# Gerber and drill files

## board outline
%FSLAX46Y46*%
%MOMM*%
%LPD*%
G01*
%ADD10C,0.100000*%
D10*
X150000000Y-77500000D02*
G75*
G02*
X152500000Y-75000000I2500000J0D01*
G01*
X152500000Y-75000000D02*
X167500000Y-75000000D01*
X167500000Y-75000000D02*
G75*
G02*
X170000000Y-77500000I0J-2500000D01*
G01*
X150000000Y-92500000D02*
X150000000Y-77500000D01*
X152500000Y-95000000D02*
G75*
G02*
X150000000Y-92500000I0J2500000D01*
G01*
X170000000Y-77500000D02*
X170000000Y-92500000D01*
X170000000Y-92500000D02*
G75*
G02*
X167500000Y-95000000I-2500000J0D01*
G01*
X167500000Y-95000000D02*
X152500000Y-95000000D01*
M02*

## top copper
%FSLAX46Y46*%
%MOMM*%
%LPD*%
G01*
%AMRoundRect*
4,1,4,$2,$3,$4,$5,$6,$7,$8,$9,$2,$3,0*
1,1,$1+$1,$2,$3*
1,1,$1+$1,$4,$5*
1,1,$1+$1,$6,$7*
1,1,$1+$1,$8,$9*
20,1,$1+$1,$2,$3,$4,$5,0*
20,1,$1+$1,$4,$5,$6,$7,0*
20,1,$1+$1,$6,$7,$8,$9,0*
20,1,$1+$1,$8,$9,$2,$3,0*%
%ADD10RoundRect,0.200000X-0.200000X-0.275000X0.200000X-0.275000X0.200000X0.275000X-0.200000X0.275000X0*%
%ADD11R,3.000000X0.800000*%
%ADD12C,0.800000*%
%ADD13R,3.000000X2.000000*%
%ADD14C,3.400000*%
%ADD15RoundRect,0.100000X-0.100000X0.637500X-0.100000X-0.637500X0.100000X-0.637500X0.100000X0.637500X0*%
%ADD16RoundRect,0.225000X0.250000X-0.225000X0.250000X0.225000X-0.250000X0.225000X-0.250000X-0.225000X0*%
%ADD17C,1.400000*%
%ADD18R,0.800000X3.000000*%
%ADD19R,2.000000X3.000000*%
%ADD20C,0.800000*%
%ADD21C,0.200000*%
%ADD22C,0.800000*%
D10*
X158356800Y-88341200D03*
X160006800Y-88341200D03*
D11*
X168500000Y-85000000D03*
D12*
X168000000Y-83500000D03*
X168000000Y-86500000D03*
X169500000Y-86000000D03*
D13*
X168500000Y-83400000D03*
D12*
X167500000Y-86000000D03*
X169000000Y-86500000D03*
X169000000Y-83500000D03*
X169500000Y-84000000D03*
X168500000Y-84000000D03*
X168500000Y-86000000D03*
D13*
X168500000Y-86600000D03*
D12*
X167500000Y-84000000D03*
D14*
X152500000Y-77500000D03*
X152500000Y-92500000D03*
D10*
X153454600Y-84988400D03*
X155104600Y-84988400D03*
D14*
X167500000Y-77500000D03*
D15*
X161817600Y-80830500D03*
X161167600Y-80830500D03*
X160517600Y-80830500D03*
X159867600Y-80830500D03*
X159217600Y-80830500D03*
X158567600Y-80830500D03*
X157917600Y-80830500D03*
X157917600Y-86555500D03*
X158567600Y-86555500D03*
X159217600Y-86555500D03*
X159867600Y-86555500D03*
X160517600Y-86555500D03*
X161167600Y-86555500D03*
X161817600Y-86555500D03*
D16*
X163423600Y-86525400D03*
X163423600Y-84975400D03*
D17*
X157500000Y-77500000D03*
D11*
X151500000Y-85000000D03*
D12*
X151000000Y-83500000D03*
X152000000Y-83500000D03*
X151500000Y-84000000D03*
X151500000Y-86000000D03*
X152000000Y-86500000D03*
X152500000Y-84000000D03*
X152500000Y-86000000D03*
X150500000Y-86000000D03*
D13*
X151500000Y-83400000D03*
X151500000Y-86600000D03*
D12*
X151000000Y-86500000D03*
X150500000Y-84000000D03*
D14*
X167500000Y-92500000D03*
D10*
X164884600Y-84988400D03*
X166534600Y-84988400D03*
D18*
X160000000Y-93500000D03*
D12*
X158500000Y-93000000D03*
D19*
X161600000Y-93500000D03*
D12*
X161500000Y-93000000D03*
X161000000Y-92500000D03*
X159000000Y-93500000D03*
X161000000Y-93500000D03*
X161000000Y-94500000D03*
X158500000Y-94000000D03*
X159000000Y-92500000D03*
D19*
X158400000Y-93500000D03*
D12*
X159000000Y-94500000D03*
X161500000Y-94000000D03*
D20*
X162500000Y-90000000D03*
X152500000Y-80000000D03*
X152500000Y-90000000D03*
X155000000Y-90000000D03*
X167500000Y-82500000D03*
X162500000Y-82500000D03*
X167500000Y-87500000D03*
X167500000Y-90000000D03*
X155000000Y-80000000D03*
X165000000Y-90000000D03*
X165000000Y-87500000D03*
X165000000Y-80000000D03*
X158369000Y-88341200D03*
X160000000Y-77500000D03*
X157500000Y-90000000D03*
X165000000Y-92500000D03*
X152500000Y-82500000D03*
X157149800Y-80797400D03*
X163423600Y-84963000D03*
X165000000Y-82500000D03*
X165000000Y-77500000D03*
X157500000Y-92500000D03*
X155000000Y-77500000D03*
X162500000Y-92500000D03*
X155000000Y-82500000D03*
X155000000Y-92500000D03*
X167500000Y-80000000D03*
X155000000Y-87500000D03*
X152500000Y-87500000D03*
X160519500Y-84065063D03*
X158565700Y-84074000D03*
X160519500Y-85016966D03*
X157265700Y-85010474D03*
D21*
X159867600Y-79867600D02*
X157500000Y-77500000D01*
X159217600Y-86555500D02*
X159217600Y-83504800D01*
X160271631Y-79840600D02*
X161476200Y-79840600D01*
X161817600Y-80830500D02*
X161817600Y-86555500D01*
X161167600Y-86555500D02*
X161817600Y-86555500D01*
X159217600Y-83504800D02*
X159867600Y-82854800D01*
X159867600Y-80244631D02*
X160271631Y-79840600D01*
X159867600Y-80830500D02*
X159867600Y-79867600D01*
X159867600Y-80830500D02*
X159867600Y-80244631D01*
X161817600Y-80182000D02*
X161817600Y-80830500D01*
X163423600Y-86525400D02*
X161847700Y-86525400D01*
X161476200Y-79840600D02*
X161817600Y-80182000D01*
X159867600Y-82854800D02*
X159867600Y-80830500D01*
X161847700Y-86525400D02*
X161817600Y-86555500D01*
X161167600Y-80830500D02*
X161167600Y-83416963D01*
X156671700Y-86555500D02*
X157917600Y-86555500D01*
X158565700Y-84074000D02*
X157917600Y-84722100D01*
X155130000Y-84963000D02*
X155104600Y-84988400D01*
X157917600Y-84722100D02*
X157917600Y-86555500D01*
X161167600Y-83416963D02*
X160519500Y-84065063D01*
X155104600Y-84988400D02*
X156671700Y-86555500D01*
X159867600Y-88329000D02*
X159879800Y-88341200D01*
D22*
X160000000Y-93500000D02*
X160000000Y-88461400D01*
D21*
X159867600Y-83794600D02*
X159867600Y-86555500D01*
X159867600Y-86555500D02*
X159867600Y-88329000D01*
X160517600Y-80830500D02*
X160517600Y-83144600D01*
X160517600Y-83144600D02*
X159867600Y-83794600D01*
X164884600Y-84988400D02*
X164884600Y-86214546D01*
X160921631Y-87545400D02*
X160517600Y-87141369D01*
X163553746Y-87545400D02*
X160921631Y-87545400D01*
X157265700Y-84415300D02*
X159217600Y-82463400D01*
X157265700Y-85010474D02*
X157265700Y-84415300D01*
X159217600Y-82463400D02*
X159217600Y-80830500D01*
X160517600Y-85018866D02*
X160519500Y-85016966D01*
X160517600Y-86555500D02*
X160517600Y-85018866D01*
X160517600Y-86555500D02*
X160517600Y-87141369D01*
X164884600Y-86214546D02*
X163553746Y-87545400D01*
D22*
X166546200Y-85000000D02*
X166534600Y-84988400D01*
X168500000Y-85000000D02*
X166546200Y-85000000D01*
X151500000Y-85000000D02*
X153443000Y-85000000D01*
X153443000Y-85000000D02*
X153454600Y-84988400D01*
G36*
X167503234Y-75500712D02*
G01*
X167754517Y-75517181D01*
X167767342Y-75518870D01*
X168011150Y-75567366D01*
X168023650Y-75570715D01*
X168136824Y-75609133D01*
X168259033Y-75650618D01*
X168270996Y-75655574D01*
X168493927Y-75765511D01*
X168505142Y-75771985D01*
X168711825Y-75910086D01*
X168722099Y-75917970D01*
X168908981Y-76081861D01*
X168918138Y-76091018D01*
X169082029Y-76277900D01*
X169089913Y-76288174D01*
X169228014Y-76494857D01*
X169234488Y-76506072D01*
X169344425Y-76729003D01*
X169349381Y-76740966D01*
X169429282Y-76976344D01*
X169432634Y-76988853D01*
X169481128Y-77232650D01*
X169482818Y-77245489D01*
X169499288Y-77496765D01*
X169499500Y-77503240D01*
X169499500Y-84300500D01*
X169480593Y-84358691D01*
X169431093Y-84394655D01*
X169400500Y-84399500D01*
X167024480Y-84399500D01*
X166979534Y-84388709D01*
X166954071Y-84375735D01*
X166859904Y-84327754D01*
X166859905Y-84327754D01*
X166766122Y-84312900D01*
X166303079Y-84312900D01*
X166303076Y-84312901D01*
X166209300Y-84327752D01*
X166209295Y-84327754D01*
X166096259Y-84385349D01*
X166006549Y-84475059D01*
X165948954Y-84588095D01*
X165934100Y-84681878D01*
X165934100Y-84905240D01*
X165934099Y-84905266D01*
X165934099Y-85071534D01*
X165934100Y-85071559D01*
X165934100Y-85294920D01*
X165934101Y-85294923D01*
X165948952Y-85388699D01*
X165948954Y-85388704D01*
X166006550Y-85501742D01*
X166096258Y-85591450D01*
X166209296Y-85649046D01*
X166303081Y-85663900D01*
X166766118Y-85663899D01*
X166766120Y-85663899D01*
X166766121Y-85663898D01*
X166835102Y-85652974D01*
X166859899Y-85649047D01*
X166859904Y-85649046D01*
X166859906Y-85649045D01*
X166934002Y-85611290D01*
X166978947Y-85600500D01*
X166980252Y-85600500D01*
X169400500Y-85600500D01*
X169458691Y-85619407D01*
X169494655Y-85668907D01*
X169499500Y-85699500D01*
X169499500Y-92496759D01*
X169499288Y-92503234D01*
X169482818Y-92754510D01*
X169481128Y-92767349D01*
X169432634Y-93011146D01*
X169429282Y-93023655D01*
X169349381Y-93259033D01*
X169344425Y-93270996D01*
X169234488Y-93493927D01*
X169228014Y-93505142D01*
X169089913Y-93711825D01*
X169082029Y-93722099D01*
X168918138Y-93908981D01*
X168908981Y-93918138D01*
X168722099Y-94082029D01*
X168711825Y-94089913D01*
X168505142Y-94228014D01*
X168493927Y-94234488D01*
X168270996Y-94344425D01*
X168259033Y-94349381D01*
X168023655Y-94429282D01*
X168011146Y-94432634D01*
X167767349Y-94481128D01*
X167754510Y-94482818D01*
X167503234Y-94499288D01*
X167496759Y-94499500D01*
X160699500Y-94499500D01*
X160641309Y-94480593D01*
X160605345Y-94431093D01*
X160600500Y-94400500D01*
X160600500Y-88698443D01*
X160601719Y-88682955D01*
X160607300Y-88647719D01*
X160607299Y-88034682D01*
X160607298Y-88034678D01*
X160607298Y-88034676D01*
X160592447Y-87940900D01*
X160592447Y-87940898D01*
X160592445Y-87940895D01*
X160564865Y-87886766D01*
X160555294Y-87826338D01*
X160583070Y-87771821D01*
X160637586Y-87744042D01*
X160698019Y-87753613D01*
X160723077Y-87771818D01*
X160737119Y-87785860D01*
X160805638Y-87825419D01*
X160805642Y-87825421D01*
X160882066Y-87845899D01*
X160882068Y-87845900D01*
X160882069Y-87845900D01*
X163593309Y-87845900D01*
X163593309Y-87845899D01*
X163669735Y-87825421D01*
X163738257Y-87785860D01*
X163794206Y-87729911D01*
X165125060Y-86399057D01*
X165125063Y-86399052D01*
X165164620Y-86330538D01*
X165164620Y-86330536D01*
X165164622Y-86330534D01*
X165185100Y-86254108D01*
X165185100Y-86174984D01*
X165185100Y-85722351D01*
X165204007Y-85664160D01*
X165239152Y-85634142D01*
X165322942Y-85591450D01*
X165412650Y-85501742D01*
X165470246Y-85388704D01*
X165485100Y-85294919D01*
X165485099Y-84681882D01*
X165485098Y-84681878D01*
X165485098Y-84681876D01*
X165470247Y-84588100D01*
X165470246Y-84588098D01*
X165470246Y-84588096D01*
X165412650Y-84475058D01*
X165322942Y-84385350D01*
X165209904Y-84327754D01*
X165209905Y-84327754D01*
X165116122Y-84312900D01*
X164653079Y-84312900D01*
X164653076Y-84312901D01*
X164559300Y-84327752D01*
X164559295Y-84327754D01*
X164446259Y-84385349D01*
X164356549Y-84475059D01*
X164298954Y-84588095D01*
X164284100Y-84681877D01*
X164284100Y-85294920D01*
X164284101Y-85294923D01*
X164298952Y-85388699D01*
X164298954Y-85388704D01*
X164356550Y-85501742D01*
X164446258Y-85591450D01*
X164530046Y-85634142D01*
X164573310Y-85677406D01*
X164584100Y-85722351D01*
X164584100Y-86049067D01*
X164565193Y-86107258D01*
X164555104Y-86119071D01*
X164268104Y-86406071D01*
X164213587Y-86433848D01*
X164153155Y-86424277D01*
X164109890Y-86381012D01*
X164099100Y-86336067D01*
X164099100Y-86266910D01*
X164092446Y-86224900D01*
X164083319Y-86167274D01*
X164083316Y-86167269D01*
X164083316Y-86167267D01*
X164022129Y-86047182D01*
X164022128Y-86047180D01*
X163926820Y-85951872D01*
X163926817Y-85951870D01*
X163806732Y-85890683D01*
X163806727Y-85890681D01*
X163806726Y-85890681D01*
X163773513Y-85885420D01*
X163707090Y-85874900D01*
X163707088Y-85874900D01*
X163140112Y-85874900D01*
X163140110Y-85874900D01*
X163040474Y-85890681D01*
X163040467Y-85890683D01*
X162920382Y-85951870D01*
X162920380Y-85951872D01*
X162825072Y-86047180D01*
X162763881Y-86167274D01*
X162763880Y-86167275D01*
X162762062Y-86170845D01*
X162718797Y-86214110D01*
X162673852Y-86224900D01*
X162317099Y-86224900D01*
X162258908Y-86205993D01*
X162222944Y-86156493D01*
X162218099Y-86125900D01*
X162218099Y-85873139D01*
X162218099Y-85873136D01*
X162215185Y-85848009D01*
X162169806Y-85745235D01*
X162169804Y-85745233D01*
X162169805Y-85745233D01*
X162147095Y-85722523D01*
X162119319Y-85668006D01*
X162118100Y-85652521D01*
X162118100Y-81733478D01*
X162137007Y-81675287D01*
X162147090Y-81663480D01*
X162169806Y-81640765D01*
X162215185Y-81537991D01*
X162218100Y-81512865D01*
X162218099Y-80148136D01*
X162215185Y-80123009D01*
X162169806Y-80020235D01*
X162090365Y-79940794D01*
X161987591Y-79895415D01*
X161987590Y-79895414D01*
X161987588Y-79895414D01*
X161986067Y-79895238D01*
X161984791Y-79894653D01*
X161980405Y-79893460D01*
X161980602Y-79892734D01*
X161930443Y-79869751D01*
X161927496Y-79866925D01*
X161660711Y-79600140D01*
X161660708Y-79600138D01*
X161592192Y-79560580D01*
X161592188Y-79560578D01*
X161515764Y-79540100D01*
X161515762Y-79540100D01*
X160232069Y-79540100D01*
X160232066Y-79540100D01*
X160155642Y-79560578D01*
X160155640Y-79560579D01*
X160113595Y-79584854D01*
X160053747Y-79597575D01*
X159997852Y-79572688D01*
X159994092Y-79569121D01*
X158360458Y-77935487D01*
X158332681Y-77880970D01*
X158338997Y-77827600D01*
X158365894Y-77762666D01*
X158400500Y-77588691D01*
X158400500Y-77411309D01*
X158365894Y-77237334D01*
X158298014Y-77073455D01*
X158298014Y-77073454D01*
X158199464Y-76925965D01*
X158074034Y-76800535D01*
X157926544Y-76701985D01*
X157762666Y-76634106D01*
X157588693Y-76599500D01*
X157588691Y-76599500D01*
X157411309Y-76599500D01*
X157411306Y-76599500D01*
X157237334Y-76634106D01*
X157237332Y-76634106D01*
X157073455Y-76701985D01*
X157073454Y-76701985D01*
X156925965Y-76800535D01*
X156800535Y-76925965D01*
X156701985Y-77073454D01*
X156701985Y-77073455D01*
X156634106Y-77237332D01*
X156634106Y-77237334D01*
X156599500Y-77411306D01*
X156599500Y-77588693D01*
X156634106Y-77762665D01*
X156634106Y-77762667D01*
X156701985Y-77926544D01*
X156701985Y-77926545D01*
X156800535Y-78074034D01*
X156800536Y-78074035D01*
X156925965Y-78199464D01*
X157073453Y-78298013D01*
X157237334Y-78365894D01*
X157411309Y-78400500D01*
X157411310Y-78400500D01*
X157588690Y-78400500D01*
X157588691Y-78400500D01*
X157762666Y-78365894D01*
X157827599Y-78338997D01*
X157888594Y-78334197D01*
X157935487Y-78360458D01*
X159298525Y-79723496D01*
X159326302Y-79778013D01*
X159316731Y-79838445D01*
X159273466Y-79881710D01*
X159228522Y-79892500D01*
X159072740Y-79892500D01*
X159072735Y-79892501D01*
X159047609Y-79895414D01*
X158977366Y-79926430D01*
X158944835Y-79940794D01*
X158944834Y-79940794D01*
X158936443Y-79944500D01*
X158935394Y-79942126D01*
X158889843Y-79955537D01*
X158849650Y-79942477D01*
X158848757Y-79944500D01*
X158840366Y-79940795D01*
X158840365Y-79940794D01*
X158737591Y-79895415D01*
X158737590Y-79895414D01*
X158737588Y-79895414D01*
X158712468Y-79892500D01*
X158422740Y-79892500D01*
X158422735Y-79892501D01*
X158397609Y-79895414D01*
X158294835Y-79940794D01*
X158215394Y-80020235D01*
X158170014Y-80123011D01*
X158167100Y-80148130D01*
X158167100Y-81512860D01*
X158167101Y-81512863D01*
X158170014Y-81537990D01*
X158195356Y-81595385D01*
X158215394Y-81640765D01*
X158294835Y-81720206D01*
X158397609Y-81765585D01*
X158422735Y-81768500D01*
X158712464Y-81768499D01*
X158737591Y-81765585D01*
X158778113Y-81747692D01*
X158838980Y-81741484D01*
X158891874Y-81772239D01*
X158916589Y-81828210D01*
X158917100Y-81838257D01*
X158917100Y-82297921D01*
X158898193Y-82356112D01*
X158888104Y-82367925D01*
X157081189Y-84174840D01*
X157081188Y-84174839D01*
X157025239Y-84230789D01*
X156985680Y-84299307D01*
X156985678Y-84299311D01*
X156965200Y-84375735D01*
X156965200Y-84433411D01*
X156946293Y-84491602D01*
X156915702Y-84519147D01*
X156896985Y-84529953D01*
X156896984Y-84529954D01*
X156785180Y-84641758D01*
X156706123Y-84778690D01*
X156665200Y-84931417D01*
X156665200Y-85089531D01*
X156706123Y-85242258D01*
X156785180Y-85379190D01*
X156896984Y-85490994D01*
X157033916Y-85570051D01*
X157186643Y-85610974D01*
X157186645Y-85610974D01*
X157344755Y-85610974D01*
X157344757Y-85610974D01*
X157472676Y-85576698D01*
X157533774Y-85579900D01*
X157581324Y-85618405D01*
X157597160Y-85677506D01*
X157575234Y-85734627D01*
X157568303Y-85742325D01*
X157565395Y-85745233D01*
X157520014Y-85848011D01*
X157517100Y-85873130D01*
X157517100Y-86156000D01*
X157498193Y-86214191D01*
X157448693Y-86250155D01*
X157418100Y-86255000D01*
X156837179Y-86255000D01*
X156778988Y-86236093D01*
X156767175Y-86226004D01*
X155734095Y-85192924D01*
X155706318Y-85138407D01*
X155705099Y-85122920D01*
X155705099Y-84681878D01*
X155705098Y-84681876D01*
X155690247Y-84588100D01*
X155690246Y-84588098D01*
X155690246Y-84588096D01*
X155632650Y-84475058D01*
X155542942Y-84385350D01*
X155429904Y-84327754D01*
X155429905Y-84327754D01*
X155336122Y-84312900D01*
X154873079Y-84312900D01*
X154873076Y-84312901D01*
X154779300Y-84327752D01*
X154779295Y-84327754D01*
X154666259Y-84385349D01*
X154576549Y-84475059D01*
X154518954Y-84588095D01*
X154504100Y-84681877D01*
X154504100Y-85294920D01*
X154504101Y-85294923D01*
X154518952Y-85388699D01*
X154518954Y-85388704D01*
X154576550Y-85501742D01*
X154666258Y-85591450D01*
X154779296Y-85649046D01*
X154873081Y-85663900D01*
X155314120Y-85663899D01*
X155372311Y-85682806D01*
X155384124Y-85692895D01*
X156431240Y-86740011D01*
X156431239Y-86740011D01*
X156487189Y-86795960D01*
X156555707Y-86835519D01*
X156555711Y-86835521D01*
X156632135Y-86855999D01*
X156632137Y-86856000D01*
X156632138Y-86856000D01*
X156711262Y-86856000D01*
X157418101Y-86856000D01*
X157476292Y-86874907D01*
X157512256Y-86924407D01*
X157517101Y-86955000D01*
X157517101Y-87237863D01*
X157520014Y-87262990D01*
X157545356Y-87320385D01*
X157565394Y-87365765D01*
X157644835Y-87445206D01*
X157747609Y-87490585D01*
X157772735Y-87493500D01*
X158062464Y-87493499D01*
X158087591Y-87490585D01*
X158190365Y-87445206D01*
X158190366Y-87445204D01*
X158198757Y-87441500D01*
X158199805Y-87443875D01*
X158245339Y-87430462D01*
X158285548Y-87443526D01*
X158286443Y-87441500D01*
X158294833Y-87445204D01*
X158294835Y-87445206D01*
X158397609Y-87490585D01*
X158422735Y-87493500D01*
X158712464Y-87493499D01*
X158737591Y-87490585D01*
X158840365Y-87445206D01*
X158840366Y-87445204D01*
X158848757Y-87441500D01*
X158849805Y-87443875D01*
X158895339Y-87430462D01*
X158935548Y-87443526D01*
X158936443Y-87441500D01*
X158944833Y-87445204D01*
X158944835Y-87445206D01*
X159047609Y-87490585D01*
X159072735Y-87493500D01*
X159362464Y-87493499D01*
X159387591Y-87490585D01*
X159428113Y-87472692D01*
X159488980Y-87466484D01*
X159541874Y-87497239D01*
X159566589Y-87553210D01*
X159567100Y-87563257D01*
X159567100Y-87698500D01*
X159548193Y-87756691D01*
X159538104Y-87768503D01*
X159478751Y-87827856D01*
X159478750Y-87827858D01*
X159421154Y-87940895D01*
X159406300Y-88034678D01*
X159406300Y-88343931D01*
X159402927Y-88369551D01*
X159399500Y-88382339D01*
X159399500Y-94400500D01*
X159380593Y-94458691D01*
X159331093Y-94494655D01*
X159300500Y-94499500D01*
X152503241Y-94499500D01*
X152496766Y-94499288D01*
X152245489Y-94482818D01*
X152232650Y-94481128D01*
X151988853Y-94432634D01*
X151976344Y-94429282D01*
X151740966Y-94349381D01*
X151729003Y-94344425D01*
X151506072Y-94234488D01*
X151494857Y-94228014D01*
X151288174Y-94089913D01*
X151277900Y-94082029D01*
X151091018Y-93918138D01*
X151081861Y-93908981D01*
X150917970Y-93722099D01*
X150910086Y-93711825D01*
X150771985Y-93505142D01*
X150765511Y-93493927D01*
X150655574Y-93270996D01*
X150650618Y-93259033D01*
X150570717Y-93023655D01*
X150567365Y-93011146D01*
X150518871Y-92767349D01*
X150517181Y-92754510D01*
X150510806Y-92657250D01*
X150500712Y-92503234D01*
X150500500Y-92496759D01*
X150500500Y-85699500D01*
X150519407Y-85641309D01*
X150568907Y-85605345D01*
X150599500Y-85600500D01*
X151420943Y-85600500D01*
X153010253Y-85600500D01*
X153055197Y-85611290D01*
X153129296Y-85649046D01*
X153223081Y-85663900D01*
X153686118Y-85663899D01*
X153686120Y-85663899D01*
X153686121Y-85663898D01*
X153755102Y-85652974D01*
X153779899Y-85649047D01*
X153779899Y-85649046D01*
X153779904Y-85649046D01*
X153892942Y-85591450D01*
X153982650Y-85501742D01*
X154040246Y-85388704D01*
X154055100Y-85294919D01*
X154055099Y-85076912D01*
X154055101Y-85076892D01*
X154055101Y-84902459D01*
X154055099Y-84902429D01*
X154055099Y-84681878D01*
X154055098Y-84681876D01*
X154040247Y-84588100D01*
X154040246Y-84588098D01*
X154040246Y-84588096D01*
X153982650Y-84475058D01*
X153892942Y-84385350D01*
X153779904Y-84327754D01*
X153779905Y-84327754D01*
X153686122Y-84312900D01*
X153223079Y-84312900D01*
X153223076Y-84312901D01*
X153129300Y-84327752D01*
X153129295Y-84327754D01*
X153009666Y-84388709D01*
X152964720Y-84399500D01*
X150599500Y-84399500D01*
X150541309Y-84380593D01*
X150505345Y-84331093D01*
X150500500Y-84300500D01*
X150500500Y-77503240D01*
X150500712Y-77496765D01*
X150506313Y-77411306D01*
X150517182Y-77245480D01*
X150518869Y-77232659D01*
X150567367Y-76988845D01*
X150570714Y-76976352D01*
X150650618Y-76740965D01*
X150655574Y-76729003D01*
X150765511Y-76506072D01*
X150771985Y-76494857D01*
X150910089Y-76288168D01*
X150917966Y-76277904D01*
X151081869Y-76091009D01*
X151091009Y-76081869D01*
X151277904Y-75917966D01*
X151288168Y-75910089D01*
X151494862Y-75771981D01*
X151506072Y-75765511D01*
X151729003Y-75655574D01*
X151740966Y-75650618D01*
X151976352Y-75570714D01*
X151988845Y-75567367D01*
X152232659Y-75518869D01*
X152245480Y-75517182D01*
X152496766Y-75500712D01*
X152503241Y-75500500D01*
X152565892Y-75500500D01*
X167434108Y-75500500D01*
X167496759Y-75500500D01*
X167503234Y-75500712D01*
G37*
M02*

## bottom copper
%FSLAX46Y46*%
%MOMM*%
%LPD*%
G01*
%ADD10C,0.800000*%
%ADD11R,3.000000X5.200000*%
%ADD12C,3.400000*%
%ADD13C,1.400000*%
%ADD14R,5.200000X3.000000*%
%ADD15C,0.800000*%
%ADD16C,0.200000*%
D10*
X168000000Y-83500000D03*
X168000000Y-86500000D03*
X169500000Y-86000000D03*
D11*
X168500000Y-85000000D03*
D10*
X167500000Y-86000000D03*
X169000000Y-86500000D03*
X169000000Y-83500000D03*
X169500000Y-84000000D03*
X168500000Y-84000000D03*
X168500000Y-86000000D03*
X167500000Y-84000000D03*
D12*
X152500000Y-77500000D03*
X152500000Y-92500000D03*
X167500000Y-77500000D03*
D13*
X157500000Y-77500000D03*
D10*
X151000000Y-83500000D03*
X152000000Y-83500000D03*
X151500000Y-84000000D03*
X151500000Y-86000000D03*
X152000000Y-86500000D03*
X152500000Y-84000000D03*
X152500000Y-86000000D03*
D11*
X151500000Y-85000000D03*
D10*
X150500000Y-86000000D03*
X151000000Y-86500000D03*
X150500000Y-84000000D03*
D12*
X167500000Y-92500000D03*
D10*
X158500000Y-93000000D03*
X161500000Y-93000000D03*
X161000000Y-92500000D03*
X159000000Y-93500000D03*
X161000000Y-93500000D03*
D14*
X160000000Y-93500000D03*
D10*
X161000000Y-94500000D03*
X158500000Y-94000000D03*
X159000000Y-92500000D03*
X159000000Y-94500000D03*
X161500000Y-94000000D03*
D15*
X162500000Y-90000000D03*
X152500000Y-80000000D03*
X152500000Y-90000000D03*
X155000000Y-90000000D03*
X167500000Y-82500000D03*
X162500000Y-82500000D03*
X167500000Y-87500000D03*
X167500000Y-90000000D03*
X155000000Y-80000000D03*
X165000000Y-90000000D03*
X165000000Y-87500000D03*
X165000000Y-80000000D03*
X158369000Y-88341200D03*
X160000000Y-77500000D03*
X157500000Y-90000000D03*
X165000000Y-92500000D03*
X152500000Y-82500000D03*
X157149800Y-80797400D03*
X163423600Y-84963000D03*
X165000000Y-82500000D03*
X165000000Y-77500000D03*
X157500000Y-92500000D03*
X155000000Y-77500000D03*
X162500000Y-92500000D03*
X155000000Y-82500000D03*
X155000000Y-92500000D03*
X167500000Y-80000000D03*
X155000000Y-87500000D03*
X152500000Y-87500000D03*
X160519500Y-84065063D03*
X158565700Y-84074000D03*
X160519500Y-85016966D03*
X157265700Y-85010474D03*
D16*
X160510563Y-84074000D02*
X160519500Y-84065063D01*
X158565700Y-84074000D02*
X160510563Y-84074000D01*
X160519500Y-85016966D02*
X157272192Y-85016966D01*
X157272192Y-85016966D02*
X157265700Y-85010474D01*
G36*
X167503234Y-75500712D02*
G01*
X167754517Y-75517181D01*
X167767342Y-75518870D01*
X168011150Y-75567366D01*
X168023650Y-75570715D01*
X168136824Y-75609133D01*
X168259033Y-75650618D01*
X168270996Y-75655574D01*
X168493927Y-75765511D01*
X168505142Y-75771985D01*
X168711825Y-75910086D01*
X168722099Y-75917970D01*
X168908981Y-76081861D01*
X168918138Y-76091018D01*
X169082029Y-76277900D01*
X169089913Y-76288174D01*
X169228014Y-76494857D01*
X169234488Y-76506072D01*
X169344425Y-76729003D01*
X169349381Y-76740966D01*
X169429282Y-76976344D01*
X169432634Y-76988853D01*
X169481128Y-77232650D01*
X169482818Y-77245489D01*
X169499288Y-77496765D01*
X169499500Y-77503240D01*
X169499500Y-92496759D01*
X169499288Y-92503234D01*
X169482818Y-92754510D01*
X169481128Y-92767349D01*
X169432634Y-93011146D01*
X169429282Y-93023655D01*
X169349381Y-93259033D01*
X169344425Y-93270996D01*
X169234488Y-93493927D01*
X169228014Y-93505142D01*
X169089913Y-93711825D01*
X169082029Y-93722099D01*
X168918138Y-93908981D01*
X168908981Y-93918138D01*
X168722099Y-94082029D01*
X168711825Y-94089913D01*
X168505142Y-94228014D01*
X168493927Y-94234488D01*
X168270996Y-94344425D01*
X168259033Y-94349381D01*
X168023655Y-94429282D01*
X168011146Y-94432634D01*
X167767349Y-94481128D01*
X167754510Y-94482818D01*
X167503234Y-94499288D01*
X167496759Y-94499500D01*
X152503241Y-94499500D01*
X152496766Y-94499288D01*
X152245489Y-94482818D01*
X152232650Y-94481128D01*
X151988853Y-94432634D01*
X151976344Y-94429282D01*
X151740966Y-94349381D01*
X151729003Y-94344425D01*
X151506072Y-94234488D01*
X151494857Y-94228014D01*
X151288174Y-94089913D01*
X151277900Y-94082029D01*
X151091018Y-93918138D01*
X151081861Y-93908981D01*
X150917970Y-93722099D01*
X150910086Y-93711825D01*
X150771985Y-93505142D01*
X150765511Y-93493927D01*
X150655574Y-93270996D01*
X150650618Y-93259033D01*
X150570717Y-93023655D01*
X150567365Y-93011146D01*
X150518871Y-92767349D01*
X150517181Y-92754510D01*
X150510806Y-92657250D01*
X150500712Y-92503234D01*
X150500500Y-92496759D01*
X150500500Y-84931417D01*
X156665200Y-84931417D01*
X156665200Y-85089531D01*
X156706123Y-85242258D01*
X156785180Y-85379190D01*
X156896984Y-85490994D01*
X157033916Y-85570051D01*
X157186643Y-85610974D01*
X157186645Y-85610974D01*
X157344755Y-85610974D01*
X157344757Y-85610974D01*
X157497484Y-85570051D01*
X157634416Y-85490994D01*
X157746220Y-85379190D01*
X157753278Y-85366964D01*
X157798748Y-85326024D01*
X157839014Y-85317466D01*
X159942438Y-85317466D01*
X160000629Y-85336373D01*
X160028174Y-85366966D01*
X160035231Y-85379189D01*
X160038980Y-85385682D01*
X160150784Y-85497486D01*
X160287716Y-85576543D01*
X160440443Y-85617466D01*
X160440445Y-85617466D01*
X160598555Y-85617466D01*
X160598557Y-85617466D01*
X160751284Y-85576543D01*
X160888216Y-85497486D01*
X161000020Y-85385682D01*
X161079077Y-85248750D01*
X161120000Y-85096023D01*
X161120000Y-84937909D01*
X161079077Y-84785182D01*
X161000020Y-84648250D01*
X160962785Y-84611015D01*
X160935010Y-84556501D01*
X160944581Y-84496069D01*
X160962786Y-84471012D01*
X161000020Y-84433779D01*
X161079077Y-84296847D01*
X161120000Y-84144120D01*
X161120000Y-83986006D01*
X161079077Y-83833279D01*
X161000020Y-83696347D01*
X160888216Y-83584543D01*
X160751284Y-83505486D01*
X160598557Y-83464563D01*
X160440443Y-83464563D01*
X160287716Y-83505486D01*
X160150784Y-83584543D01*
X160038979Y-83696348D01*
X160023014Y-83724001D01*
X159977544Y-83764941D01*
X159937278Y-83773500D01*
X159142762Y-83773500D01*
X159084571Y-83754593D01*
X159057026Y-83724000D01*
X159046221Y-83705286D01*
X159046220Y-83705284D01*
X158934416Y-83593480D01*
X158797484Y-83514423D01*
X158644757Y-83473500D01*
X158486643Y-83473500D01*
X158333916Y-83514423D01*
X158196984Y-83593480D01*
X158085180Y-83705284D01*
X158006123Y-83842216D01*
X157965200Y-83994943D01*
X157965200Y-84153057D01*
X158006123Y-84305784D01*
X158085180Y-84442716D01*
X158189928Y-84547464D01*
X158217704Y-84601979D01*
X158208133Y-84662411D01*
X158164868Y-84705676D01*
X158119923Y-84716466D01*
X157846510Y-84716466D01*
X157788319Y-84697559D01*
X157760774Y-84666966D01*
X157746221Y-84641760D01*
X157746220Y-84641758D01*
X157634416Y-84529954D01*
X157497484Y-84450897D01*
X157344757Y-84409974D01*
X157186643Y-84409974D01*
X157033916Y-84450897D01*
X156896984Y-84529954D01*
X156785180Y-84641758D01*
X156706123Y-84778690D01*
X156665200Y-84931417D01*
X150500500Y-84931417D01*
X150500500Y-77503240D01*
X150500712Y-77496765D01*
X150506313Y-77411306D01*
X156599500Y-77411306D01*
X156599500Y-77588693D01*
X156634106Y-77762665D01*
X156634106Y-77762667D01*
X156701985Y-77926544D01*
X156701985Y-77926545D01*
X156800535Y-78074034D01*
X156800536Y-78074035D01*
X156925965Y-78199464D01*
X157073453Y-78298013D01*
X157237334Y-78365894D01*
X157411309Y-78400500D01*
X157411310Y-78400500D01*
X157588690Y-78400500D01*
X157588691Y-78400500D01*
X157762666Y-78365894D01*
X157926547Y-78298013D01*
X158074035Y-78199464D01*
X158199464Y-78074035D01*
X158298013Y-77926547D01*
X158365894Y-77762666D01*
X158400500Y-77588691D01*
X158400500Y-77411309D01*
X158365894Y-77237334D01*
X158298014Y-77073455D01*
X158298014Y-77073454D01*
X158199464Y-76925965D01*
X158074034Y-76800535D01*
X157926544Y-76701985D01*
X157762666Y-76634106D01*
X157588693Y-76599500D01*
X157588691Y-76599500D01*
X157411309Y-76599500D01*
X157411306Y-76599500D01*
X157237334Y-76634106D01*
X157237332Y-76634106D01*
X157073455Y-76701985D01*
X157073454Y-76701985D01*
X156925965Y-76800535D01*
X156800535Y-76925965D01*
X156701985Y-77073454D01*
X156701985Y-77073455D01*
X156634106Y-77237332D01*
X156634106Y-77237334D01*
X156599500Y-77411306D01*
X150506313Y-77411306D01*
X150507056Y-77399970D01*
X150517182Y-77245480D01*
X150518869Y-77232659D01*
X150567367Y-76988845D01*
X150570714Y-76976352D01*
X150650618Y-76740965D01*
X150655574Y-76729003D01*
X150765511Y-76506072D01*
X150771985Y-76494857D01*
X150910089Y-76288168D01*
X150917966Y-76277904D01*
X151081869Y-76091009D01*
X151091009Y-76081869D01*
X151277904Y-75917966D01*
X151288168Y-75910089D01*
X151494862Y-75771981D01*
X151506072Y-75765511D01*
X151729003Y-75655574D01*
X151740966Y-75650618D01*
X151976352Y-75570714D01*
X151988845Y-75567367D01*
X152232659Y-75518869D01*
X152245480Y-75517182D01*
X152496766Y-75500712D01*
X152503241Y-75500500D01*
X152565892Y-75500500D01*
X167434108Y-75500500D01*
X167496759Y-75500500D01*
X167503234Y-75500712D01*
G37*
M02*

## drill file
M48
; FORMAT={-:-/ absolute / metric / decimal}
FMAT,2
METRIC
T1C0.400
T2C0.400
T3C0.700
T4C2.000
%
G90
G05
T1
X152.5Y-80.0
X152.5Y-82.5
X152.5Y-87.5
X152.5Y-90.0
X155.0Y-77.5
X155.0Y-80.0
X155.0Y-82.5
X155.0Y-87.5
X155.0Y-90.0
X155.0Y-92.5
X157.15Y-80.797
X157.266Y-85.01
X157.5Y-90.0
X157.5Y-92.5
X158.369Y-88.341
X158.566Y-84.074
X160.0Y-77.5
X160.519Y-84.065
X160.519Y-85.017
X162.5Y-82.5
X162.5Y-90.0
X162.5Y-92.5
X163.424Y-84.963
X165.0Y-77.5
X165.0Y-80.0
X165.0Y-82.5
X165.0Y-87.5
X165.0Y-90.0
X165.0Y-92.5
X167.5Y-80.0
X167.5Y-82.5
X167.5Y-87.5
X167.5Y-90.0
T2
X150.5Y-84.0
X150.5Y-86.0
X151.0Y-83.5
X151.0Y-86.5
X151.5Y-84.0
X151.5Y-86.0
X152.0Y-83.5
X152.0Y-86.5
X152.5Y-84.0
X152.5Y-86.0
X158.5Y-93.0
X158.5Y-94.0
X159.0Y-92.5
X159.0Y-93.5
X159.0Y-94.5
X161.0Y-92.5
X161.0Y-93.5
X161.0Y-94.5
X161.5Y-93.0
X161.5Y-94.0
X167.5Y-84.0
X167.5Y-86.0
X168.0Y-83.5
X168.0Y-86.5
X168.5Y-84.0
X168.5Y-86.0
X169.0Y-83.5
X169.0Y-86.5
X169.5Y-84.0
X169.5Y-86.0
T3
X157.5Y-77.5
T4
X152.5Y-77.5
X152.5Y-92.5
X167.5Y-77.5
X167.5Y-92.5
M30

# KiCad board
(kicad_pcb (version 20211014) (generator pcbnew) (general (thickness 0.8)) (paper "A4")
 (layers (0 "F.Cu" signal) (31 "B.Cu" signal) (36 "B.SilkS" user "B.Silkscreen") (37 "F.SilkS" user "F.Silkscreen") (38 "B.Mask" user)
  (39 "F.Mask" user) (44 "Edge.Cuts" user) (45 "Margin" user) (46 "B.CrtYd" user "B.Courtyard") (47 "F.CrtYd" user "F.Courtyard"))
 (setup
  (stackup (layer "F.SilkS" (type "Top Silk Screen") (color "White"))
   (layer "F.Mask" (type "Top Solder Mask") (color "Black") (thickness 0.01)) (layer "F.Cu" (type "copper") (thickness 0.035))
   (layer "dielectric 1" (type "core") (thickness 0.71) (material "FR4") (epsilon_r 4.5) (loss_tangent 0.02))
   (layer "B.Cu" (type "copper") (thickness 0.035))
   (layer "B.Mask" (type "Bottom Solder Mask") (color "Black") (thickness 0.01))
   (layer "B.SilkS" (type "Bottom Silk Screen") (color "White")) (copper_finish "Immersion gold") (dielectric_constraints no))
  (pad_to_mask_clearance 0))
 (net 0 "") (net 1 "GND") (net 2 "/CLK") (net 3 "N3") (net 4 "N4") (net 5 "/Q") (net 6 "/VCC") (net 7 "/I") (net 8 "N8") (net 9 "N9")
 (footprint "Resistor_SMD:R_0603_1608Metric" (layer "F.Cu") (at 159.1818 88.3412)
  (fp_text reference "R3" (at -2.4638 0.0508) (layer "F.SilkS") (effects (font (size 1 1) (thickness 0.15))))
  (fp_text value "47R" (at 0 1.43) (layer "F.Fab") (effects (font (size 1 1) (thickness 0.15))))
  (pad "1" smd roundrect (at -0.825 0) (size 0.8 0.95) (layers "F.Cu" "F.Paste" "F.Mask") (roundrect_rratio 0.25) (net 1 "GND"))
  (pad "2" smd roundrect (at 0.825 0) (size 0.8 0.95) (layers "F.Cu" "F.Paste" "F.Mask") (roundrect_rratio 0.25) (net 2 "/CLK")))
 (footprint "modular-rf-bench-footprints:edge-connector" (layer "F.Cu") (at 170 85)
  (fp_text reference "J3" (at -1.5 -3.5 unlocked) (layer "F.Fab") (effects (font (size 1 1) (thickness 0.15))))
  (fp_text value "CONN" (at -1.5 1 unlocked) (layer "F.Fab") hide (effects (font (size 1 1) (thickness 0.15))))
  (pad "1" smd rect (at -1.5 0) (size 3 0.8) (layers "F.Cu") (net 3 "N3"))
  (pad "2" thru_hole circle (at -2 -1.5) (size 0.8 0.8) (drill 0.4) (layers *.Cu) (remove_unused_layers) (keep_end_layers) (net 1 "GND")
   (zone_connect 2))
  (pad "2" thru_hole circle (at -2 1.5) (size 0.8 0.8) (drill 0.4) (layers *.Cu) (remove_unused_layers) (keep_end_layers) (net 1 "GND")
   (zone_connect 2))
  (pad "2" thru_hole circle (at -0.5 1) (size 0.8 0.8) (drill 0.4) (layers *.Cu) (remove_unused_layers) (keep_end_layers) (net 1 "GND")
   (zone_connect 2))
  (pad "2" smd rect (at -1.5 -1.6) (size 3 2) (layers "F.Cu") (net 1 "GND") (zone_connect 2))
  (pad "2" smd rect (at -1.5 0) (size 3 5.2) (layers "B.Cu") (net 1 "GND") (zone_connect 2))
  (pad "2" thru_hole circle (at -2.5 1) (size 0.8 0.8) (drill 0.4) (layers *.Cu) (remove_unused_layers) (keep_end_layers) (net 1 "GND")
   (zone_connect 2))
  (pad "2" thru_hole circle (at -1 1.5) (size 0.8 0.8) (drill 0.4) (layers *.Cu) (remove_unused_layers) (keep_end_layers) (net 1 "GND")
   (zone_connect 2))
  (pad "2" thru_hole circle (at -1 -1.5) (size 0.8 0.8) (drill 0.4) (layers *.Cu) (remove_unused_layers) (keep_end_layers) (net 1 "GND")
   (zone_connect 2))
  (pad "2" thru_hole circle (at -0.5 -1) (size 0.8 0.8) (drill 0.4) (layers *.Cu) (remove_unused_layers) (keep_end_layers) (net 1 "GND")
   (zone_connect 2))
  (pad "2" thru_hole circle (at -1.5 -1) (size 0.8 0.8) (drill 0.4) (layers *.Cu) (remove_unused_layers) (keep_end_layers) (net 1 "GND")
   (zone_connect 2))
  (pad "2" thru_hole circle (at -1.5 1) (size 0.8 0.8) (drill 0.4) (layers *.Cu) (remove_unused_layers) (keep_end_layers) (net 1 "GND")
   (zone_connect 2))
  (pad "2" smd rect (at -1.5 1.6) (size 3 2) (layers "F.Cu") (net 1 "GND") (zone_connect 2))
  (pad "2" thru_hole circle (at -2.5 -1) (size 0.8 0.8) (drill 0.4) (layers *.Cu) (remove_unused_layers) (keep_end_layers) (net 1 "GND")
   (zone_connect 2)))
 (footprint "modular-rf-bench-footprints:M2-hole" (layer "F.Cu") (at 152.5 77.5)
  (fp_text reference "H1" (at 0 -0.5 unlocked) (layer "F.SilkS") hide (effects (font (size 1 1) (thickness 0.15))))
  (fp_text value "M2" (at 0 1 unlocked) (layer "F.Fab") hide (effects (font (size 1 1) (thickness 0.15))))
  (pad "1" thru_hole circle (at 0 0) (size 3.4 3.4) (drill 2) (layers *.Cu *.Mask) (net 1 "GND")))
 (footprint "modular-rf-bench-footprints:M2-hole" (layer "F.Cu") (at 152.5 92.5)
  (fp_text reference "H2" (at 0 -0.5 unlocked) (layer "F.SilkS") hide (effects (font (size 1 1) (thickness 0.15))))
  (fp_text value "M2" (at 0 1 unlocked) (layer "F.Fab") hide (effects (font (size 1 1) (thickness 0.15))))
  (pad "1" thru_hole circle (at 0 0) (size 3.4 3.4) (drill 2) (layers *.Cu *.Mask) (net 1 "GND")))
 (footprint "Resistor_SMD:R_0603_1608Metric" (layer "F.Cu") (at 154.2796 84.9884)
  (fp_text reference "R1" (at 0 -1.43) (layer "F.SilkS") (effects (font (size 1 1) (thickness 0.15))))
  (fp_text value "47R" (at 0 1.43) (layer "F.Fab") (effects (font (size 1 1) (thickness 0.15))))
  (pad "1" smd roundrect (at -0.825 0) (size 0.8 0.95) (layers "F.Cu" "F.Paste" "F.Mask") (roundrect_rratio 0.25) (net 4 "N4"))
  (pad "2" smd roundrect (at 0.825 0) (size 0.8 0.95) (layers "F.Cu" "F.Paste" "F.Mask") (roundrect_rratio 0.25) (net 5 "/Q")))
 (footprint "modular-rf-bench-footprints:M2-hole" (layer "F.Cu") (at 167.5 77.5)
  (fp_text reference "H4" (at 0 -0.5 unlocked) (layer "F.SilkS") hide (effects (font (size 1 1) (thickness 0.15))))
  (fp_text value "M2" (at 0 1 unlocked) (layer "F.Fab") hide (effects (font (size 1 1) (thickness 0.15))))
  (pad "1" thru_hole circle (at 0 0) (size 3.4 3.4) (drill 2) (layers *.Cu *.Mask) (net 1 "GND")))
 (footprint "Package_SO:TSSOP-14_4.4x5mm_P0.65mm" (layer "F.Cu") (at 159.8676 83.693 -90)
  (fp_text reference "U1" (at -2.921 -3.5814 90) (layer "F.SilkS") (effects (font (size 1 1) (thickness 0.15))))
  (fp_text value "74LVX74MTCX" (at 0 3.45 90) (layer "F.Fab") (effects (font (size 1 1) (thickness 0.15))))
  (pad "1" smd roundrect (at -2.8625 -1.95 270) (size 1.475 0.4) (layers "F.Cu" "F.Paste" "F.Mask") (roundrect_rratio 0.25) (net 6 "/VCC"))
  (pad "2" smd roundrect (at -2.8625 -1.3 270) (size 1.475 0.4) (layers "F.Cu" "F.Paste" "F.Mask") (roundrect_rratio 0.25) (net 5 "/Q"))
  (pad "3" smd roundrect (at -2.8625 -0.65 270) (size 1.475 0.4) (layers "F.Cu" "F.Paste" "F.Mask") (roundrect_rratio 0.25) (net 2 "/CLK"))
  (pad "4" smd roundrect (at -2.8625 0 270) (size 1.475 0.4) (layers "F.Cu" "F.Paste" "F.Mask") (roundrect_rratio 0.25) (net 6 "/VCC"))
  (pad "5" smd roundrect (at -2.8625 0.65 270) (size 1.475 0.4) (layers "F.Cu" "F.Paste" "F.Mask") (roundrect_rratio 0.25) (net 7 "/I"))
  (pad "6" smd roundrect (at -2.8625 1.3 270) (size 1.475 0.4) (layers "F.Cu" "F.Paste" "F.Mask") (roundrect_rratio 0.25) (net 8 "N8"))
  (pad "7" smd roundrect (at -2.8625 1.95 270) (size 1.475 0.4) (layers "F.Cu" "F.Paste" "F.Mask") (roundrect_rratio 0.25) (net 1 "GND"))
  (pad "8" smd roundrect (at 2.8625 1.95 270) (size 1.475 0.4) (layers "F.Cu" "F.Paste" "F.Mask") (roundrect_rratio 0.25) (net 5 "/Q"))
  (pad "9" smd roundrect (at 2.8625 1.3 270) (size 1.475 0.4) (layers "F.Cu" "F.Paste" "F.Mask") (roundrect_rratio 0.25) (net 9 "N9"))
  (pad "10" smd roundrect (at 2.8625 0.65 270) (size 1.475 0.4) (layers "F.Cu" "F.Paste" "F.Mask") (roundrect_rratio 0.25) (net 6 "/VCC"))
  (pad "11" smd roundrect (at 2.8625 0 270) (size 1.475 0.4) (layers "F.Cu" "F.Paste" "F.Mask") (roundrect_rratio 0.25) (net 2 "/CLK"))
  (pad "12" smd roundrect (at 2.8625 -0.65 270) (size 1.475 0.4) (layers "F.Cu" "F.Paste" "F.Mask") (roundrect_rratio 0.25) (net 7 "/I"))
  (pad "13" smd roundrect (at 2.8625 -1.3 270) (size 1.475 0.4) (layers "F.Cu" "F.Paste" "F.Mask") (roundrect_rratio 0.25) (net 6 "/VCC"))
  (pad "14" smd roundrect (at 2.8625 -1.95 270) (size 1.475 0.4) (layers "F.Cu" "F.Paste" "F.Mask") (roundrect_rratio 0.25) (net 6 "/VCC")))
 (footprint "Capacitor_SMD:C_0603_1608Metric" (layer "F.Cu") (at 163.4236 85.7504 90)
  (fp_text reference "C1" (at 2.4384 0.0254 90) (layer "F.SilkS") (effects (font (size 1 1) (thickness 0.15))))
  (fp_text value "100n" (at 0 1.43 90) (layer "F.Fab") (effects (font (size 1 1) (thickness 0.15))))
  (pad "1" smd roundrect (at -0.775 0 90) (size 0.9 0.95) (layers "F.Cu" "F.Paste" "F.Mask") (roundrect_rratio 0.25) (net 6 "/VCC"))
  (pad "2" smd roundrect (at 0.775 0 90) (size 0.9 0.95) (layers "F.Cu" "F.Paste" "F.Mask") (roundrect_rratio 0.25) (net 1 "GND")))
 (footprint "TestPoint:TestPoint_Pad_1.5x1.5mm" (layer "F.Cu") (at 157.5 77.5)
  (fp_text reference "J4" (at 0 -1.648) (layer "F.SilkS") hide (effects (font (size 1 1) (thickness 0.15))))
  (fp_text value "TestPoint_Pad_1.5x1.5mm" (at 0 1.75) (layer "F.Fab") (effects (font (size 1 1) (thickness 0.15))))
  (pad "1" thru_hole circle (at 0 0) (size 1.4 1.4) (drill 0.7) (layers *.Cu *.Mask) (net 6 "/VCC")))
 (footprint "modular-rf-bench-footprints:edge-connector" (layer "F.Cu") (at 150 85 180)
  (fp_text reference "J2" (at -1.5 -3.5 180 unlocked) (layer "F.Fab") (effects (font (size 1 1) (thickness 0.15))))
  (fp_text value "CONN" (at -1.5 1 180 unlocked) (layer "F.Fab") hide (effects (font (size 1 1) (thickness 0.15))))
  (pad "1" smd rect (at -1.5 0 180) (size 3 0.8) (layers "F.Cu") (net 4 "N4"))
  (pad "2" thru_hole circle (at -1 1.5 180) (size 0.8 0.8) (drill 0.4) (layers *.Cu) (remove_unused_layers) (keep_end_layers) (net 1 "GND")
   (zone_connect 2))
  (pad "2" thru_hole circle (at -2 1.5 180) (size 0.8 0.8) (drill 0.4) (layers *.Cu) (remove_unused_layers) (keep_end_layers) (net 1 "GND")
   (zone_connect 2))
  (pad "2" thru_hole circle (at -1.5 1 180) (size 0.8 0.8) (drill 0.4) (layers *.Cu) (remove_unused_layers) (keep_end_layers) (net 1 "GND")
   (zone_connect 2))
  (pad "2" thru_hole circle (at -1.5 -1 180) (size 0.8 0.8) (drill 0.4) (layers *.Cu) (remove_unused_layers) (keep_end_layers) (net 1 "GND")
   (zone_connect 2))
  (pad "2" thru_hole circle (at -2 -1.5 180) (size 0.8 0.8) (drill 0.4) (layers *.Cu) (remove_unused_layers) (keep_end_layers) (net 1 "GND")
   (zone_connect 2))
  (pad "2" thru_hole circle (at -2.5 1 180) (size 0.8 0.8) (drill 0.4) (layers *.Cu) (remove_unused_layers) (keep_end_layers) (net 1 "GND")
   (zone_connect 2))
  (pad "2" thru_hole circle (at -2.5 -1 180) (size 0.8 0.8) (drill 0.4) (layers *.Cu) (remove_unused_layers) (keep_end_layers) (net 1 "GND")
   (zone_connect 2))
  (pad "2" smd rect (at -1.5 0 180) (size 3 5.2) (layers "B.Cu") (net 1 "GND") (zone_connect 2))
  (pad "2" thru_hole circle (at -0.5 -1 180) (size 0.8 0.8) (drill 0.4) (layers *.Cu) (remove_unused_layers) (keep_end_layers) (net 1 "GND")
   (zone_connect 2))
  (pad "2" smd rect (at -1.5 1.6 180) (size 3 2) (layers "F.Cu") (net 1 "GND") (zone_connect 2))
  (pad "2" smd rect (at -1.5 -1.6 180) (size 3 2) (layers "F.Cu") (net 1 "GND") (zone_connect 2))
  (pad "2" thru_hole circle (at -1 -1.5 180) (size 0.8 0.8) (drill 0.4) (layers *.Cu) (remove_unused_layers) (keep_end_layers) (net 1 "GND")
   (zone_connect 2))
  (pad "2" thru_hole circle (at -0.5 1 180) (size 0.8 0.8) (drill 0.4) (layers *.Cu) (remove_unused_layers) (keep_end_layers) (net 1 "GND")
   (zone_connect 2)))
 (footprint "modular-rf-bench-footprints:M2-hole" (layer "F.Cu") (at 167.5 92.5)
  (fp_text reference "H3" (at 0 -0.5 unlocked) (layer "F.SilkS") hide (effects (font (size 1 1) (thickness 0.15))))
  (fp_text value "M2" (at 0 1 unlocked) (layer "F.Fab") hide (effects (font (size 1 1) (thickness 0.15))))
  (pad "1" thru_hole circle (at 0 0) (size 3.4 3.4) (drill 2) (layers *.Cu *.Mask) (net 1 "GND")))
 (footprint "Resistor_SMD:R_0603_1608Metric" (layer "F.Cu") (at 165.7096 84.9884)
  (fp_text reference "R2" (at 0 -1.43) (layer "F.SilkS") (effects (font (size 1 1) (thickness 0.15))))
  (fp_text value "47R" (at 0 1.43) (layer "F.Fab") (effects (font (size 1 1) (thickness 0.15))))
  (pad "1" smd roundrect (at -0.825 0) (size 0.8 0.95) (layers "F.Cu" "F.Paste" "F.Mask") (roundrect_rratio 0.25) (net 7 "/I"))
  (pad "2" smd roundrect (at 0.825 0) (size 0.8 0.95) (layers "F.Cu" "F.Paste" "F.Mask") (roundrect_rratio 0.25) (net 3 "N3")))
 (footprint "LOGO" (layer "F.Cu") (at 164.25 89.5)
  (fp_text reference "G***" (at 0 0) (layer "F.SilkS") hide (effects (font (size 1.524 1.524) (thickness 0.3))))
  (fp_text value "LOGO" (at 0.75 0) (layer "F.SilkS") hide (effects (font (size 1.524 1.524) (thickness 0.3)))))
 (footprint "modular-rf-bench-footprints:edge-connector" (layer "F.Cu") (at 160 95 -90)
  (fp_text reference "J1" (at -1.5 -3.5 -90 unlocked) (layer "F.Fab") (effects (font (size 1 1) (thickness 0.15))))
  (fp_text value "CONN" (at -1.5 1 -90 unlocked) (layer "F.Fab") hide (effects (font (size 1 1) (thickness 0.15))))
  (pad "1" smd rect (at -1.5 0 270) (size 3 0.8) (layers "F.Cu") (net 2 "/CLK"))
  (pad "2" thru_hole circle (at -2 1.5 270) (size 0.8 0.8) (drill 0.4) (layers *.Cu) (remove_unused_layers) (keep_end_layers) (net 1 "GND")
   (zone_connect 2))
  (pad "2" smd rect (at -1.5 -1.6 270) (size 3 2) (layers "F.Cu") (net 1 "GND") (zone_connect 2))
  (pad "2" thru_hole circle (at -2 -1.5 270) (size 0.8 0.8) (drill 0.4) (layers *.Cu) (remove_unused_layers) (keep_end_layers) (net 1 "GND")
   (zone_connect 2))
  (pad "2" thru_hole circle (at -2.5 -1 270) (size 0.8 0.8) (drill 0.4) (layers *.Cu) (remove_unused_layers) (keep_end_layers) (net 1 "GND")
   (zone_connect 2))
  (pad "2" thru_hole circle (at -1.5 1 270) (size 0.8 0.8) (drill 0.4) (layers *.Cu) (remove_unused_layers) (keep_end_layers) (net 1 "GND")
   (zone_connect 2))
  (pad "2" thru_hole circle (at -1.5 -1 270) (size 0.8 0.8) (drill 0.4) (layers *.Cu) (remove_unused_layers) (keep_end_layers) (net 1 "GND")
   (zone_connect 2))
  (pad "2" smd rect (at -1.5 0 270) (size 3 5.2) (layers "B.Cu") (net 1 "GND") (zone_connect 2))
  (pad "2" thru_hole circle (at -0.5 -1 270) (size 0.8 0.8) (drill 0.4) (layers *.Cu) (remove_unused_layers) (keep_end_layers) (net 1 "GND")
   (zone_connect 2))
  (pad "2" thru_hole circle (at -1 1.5 270) (size 0.8 0.8) (drill 0.4) (layers *.Cu) (remove_unused_layers) (keep_end_layers) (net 1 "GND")
   (zone_connect 2))
  (pad "2" thru_hole circle (at -2.5 1 270) (size 0.8 0.8) (drill 0.4) (layers *.Cu) (remove_unused_layers) (keep_end_layers) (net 1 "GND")
   (zone_connect 2))
  (pad "2" smd rect (at -1.5 1.6 270) (size 3 2) (layers "F.Cu") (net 1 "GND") (zone_connect 2))
  (pad "2" thru_hole circle (at -0.5 1 270) (size 0.8 0.8) (drill 0.4) (layers *.Cu) (remove_unused_layers) (keep_end_layers) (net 1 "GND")
   (zone_connect 2))
  (pad "2" thru_hole circle (at -1 -1.5 270) (size 0.8 0.8) (drill 0.4) (layers *.Cu) (remove_unused_layers) (keep_end_layers) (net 1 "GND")
   (zone_connect 2)))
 (gr_arc (start 150 77.5) (mid 150.732233 75.732233) (end 152.5 75) (layer "Edge.Cuts") (width 0.1))
 (gr_line (start 152.5 75) (end 167.5 75) (layer "Edge.Cuts") (width 0.1))
 (gr_arc (start 167.5 75) (mid 169.267767 75.732233) (end 170 77.5) (layer "Edge.Cuts") (width 0.1))
 (gr_line (start 150 92.5) (end 150 77.5) (layer "Edge.Cuts") (width 0.1))
 (gr_arc (start 152.5 95) (mid 150.732233 94.267767) (end 150 92.5) (layer "Edge.Cuts") (width 0.1))
 (gr_line (start 170 77.5) (end 170 92.5) (layer "Edge.Cuts") (width 0.1))
 (gr_arc (start 170 92.5) (mid 169.267767 94.267767) (end 167.5 95) (layer "Edge.Cuts") (width 0.1))
 (gr_line (start 167.5 95) (end 152.5 95) (layer "Edge.Cuts") (width 0.1))
 (via (at 162.5 90) (size 0.8) (drill 0.4) (layers "F.Cu" "B.Cu") (free) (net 1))
 (via (at 152.5 80) (size 0.8) (drill 0.4) (layers "F.Cu" "B.Cu") (free) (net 1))
 (via (at 152.5 90) (size 0.8) (drill 0.4) (layers "F.Cu" "B.Cu") (free) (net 1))
 (via (at 155 90) (size 0.8) (drill 0.4) (layers "F.Cu" "B.Cu") (free) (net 1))
 (via (at 167.5 82.5) (size 0.8) (drill 0.4) (layers "F.Cu" "B.Cu") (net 1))
 (via (at 162.5 82.5) (size 0.8) (drill 0.4) (layers "F.Cu" "B.Cu") (free) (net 1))
 (via (at 167.5 87.5) (size 0.8) (drill 0.4) (layers "F.Cu" "B.Cu") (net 1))
 (via (at 167.5 90) (size 0.8) (drill 0.4) (layers "F.Cu" "B.Cu") (free) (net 1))
 (via (at 155 80) (size 0.8) (drill 0.4) (layers "F.Cu" "B.Cu") (free) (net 1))
 (via (at 165 90) (size 0.8) (drill 0.4) (layers "F.Cu" "B.Cu") (free) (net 1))
 (via (at 165 87.5) (size 0.8) (drill 0.4) (layers "F.Cu" "B.Cu") (free) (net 1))
 (via (at 165 80) (size 0.8) (drill 0.4) (layers "F.Cu" "B.Cu") (free) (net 1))
 (via (at 158.369 88.3412) (size 0.8) (drill 0.4) (layers "F.Cu" "B.Cu") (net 1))
 (via (at 160 77.5) (size 0.8) (drill 0.4) (layers "F.Cu" "B.Cu") (free) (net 1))
 (via (at 157.5 90) (size 0.8) (drill 0.4) (layers "F.Cu" "B.Cu") (free) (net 1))
 (via (at 165 92.5) (size 0.8) (drill 0.4) (layers "F.Cu" "B.Cu") (free) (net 1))
 (via (at 152.5 82.5) (size 0.8) (drill 0.4) (layers "F.Cu" "B.Cu") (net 1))
 (via (at 157.1498 80.7974) (size 0.8) (drill 0.4) (layers "F.Cu" "B.Cu") (free) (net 1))
 (via (at 163.4236 84.963) (size 0.8) (drill 0.4) (layers "F.Cu" "B.Cu") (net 1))
 (via (at 165 82.5) (size 0.8) (drill 0.4) (layers "F.Cu" "B.Cu") (free) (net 1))
 (via (at 165 77.5) (size 0.8) (drill 0.4) (layers "F.Cu" "B.Cu") (free) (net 1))
 (via (at 157.5 92.5) (size 0.8) (drill 0.4) (layers "F.Cu" "B.Cu") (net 1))
 (via (at 155 77.5) (size 0.8) (drill 0.4) (layers "F.Cu" "B.Cu") (free) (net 1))
 (via (at 162.5 92.5) (size 0.8) (drill 0.4) (layers "F.Cu" "B.Cu") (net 1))
 (via (at 155 82.5) (size 0.8) (drill 0.4) (layers "F.Cu" "B.Cu") (free) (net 1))
 (via (at 155 92.5) (size 0.8) (drill 0.4) (layers "F.Cu" "B.Cu") (free) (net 1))
 (via (at 167.5 80) (size 0.8) (drill 0.4) (layers "F.Cu" "B.Cu") (free) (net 1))
 (via (at 155 87.5) (size 0.8) (drill 0.4) (layers "F.Cu" "B.Cu") (free) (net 1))
 (via (at 152.5 87.5) (size 0.8) (drill 0.4) (layers "F.Cu" "B.Cu") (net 1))
 (segment (start 159.8676 79.8676) (end 157.5 77.5) (width 0.2) (layer "F.Cu") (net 6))
 (segment (start 159.2176 86.5555) (end 159.2176 83.5048) (width 0.2) (layer "F.Cu") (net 6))
 (segment (start 160.271631 79.8406) (end 161.4762 79.8406) (width 0.2) (layer "F.Cu") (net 6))
 (segment (start 161.8176 80.8305) (end 161.8176 86.5555) (width 0.2) (layer "F.Cu") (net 6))
 (segment (start 161.1676 86.5555) (end 161.8176 86.5555) (width 0.2) (layer "F.Cu") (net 6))
 (segment (start 159.2176 83.5048) (end 159.8676 82.8548) (width 0.2) (layer "F.Cu") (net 6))
 (segment (start 159.8676 80.244631) (end 160.271631 79.8406) (width 0.2) (layer "F.Cu") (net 6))
 (segment (start 159.8676 80.8305) (end 159.8676 79.8676) (width 0.2) (layer "F.Cu") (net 6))
 (segment (start 159.8676 80.8305) (end 159.8676 80.244631) (width 0.2) (layer "F.Cu") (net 6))
 (segment (start 161.8176 80.182) (end 161.8176 80.8305) (width 0.2) (layer "F.Cu") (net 6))
 (segment (start 163.4236 86.5254) (end 161.8477 86.5254) (width 0.2) (layer "F.Cu") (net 6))
 (segment (start 161.4762 79.8406) (end 161.8176 80.182) (width 0.2) (layer "F.Cu") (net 6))
 (segment (start 159.8676 82.8548) (end 159.8676 80.8305) (width 0.2) (layer "F.Cu") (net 6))
 (segment (start 161.8477 86.5254) (end 161.8176 86.5555) (width 0.2) (layer "F.Cu") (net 6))
 (segment (start 161.1676 80.8305) (end 161.1676 83.416963) (width 0.2) (layer "F.Cu") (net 5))
 (segment (start 156.6717 86.5555) (end 157.9176 86.5555) (width 0.2) (layer "F.Cu") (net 5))
 (segment (start 158.5657 84.074) (end 157.9176 84.7221) (width 0.2) (layer "F.Cu") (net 5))
 (segment (start 155.13 84.963) (end 155.1046 84.9884) (width 0.2) (layer "F.Cu") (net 5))
 (segment (start 157.9176 84.7221) (end 157.9176 86.5555) (width 0.2) (layer "F.Cu") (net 5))
 (segment (start 161.1676 83.416963) (end 160.5195 84.065063) (width 0.2) (layer "F.Cu") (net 5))
 (segment (start 155.1046 84.9884) (end 156.6717 86.5555) (width 0.2) (layer "F.Cu") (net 5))
 (via (at 160.5195 84.065063) (size 0.8) (drill 0.4) (layers "F.Cu" "B.Cu") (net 5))
 (via (at 158.5657 84.074) (size 0.8) (drill 0.4) (layers "F.Cu" "B.Cu") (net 5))
 (segment (start 160.510563 84.074) (end 160.5195 84.065063) (width 0.2) (layer "B.Cu") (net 5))
 (segment (start 158.5657 84.074) (end 160.510563 84.074) (width 0.2) (layer "B.Cu") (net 5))
 (segment (start 159.8676 88.329) (end 159.8798 88.3412) (width 0.2) (layer "F.Cu") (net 2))
 (segment (start 160 93.5) (end 160 88.4614) (width 0.8) (layer "F.Cu") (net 2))
 (segment (start 159.8676 83.7946) (end 159.8676 86.5555) (width 0.2) (layer "F.Cu") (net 2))
 (segment (start 159.8676 86.5555) (end 159.8676 88.329) (width 0.2) (layer "F.Cu") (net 2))
 (segment (start 160.5176 80.8305) (end 160.5176 83.1446) (width 0.2) (layer "F.Cu") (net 2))
 (segment (start 160.5176 83.1446) (end 159.8676 83.7946) (width 0.2) (layer "F.Cu") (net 2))
 (segment (start 164.8846 84.9884) (end 164.8846 86.214546) (width 0.2) (layer "F.Cu") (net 7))
 (segment (start 160.921631 87.5454) (end 160.5176 87.141369) (width 0.2) (layer "F.Cu") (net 7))
 (segment (start 163.553746 87.5454) (end 160.921631 87.5454) (width 0.2) (layer "F.Cu") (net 7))
 (segment (start 157.2657 84.4153) (end 159.2176 82.4634) (width 0.2) (layer "F.Cu") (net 7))
 (segment (start 157.2657 85.010474) (end 157.2657 84.4153) (width 0.2) (layer "F.Cu") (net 7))
 (segment (start 159.2176 82.4634) (end 159.2176 80.8305) (width 0.2) (layer "F.Cu") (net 7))
 (segment (start 160.5176 85.018866) (end 160.5195 85.016966) (width 0.2) (layer "F.Cu") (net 7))
 (segment (start 160.5176 86.5555) (end 160.5176 85.018866) (width 0.2) (layer "F.Cu") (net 7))
 (segment (start 160.5176 86.5555) (end 160.5176 87.141369) (width 0.2) (layer "F.Cu") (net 7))
 (segment (start 164.8846 86.214546) (end 163.553746 87.5454) (width 0.2) (layer "F.Cu") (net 7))
 (via (at 160.5195 85.016966) (size 0.8) (drill 0.4) (layers "F.Cu" "B.Cu") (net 7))
 (via (at 157.2657 85.010474) (size 0.8) (drill 0.4) (layers "F.Cu" "B.Cu") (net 7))
 (segment (start 160.5195 85.016966) (end 157.272192 85.016966) (width 0.2) (layer "B.Cu") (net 7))
 (segment (start 157.272192 85.016966) (end 157.2657 85.010474) (width 0.2) (layer "B.Cu") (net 7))
 (segment (start 166.5462 85) (end 166.5346 84.9884) (width 0.8) (layer "F.Cu") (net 3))
 (segment (start 168.5 85) (end 166.5462 85) (width 0.8) (layer "F.Cu") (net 3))
 (segment (start 151.5 85) (end 153.443 85) (width 0.8) (layer "F.Cu") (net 4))
 (segment (start 153.443 85) (end 153.4546 84.9884) (width 0.8) (layer "F.Cu") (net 4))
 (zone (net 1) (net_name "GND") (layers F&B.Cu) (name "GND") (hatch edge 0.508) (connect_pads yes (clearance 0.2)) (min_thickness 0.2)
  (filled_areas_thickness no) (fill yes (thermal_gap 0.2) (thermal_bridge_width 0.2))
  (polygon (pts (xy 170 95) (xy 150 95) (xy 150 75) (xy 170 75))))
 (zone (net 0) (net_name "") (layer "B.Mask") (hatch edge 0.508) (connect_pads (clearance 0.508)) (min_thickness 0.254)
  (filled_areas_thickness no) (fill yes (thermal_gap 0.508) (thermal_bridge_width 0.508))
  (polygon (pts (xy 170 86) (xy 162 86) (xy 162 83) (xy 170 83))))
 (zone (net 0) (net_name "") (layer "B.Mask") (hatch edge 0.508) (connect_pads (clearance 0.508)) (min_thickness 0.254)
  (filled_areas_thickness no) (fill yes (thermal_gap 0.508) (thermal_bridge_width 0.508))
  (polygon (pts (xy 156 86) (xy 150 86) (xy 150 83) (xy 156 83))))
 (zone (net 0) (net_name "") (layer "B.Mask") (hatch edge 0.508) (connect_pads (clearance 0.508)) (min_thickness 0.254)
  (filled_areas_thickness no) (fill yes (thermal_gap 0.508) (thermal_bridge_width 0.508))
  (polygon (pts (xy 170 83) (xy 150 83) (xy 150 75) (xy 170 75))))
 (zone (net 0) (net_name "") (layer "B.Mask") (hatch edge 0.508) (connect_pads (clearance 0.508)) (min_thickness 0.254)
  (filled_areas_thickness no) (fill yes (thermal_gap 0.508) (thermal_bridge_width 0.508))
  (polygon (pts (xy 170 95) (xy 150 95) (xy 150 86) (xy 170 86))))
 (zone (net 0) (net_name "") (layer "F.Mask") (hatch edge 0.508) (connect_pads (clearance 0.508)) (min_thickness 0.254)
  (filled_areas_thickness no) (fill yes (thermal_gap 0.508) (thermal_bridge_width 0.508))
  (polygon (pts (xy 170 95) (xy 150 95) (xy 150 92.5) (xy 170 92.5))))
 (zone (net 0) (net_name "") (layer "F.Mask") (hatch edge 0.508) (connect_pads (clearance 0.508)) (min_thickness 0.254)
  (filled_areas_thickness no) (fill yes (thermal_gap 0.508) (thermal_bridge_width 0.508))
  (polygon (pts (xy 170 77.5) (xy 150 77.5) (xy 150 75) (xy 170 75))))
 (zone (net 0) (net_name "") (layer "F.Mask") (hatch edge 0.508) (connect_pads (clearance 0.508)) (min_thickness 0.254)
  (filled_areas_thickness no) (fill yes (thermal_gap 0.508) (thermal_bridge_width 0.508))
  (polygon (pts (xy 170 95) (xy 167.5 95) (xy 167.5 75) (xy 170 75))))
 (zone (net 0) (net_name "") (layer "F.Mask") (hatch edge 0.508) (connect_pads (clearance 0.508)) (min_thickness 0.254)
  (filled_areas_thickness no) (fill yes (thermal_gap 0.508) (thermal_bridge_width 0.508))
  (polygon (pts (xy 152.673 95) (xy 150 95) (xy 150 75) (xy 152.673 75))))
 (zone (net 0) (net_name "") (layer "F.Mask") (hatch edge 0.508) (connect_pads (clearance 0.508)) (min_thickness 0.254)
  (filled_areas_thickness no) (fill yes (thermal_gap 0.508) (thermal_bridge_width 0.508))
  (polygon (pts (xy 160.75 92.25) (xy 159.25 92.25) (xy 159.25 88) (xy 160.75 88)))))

